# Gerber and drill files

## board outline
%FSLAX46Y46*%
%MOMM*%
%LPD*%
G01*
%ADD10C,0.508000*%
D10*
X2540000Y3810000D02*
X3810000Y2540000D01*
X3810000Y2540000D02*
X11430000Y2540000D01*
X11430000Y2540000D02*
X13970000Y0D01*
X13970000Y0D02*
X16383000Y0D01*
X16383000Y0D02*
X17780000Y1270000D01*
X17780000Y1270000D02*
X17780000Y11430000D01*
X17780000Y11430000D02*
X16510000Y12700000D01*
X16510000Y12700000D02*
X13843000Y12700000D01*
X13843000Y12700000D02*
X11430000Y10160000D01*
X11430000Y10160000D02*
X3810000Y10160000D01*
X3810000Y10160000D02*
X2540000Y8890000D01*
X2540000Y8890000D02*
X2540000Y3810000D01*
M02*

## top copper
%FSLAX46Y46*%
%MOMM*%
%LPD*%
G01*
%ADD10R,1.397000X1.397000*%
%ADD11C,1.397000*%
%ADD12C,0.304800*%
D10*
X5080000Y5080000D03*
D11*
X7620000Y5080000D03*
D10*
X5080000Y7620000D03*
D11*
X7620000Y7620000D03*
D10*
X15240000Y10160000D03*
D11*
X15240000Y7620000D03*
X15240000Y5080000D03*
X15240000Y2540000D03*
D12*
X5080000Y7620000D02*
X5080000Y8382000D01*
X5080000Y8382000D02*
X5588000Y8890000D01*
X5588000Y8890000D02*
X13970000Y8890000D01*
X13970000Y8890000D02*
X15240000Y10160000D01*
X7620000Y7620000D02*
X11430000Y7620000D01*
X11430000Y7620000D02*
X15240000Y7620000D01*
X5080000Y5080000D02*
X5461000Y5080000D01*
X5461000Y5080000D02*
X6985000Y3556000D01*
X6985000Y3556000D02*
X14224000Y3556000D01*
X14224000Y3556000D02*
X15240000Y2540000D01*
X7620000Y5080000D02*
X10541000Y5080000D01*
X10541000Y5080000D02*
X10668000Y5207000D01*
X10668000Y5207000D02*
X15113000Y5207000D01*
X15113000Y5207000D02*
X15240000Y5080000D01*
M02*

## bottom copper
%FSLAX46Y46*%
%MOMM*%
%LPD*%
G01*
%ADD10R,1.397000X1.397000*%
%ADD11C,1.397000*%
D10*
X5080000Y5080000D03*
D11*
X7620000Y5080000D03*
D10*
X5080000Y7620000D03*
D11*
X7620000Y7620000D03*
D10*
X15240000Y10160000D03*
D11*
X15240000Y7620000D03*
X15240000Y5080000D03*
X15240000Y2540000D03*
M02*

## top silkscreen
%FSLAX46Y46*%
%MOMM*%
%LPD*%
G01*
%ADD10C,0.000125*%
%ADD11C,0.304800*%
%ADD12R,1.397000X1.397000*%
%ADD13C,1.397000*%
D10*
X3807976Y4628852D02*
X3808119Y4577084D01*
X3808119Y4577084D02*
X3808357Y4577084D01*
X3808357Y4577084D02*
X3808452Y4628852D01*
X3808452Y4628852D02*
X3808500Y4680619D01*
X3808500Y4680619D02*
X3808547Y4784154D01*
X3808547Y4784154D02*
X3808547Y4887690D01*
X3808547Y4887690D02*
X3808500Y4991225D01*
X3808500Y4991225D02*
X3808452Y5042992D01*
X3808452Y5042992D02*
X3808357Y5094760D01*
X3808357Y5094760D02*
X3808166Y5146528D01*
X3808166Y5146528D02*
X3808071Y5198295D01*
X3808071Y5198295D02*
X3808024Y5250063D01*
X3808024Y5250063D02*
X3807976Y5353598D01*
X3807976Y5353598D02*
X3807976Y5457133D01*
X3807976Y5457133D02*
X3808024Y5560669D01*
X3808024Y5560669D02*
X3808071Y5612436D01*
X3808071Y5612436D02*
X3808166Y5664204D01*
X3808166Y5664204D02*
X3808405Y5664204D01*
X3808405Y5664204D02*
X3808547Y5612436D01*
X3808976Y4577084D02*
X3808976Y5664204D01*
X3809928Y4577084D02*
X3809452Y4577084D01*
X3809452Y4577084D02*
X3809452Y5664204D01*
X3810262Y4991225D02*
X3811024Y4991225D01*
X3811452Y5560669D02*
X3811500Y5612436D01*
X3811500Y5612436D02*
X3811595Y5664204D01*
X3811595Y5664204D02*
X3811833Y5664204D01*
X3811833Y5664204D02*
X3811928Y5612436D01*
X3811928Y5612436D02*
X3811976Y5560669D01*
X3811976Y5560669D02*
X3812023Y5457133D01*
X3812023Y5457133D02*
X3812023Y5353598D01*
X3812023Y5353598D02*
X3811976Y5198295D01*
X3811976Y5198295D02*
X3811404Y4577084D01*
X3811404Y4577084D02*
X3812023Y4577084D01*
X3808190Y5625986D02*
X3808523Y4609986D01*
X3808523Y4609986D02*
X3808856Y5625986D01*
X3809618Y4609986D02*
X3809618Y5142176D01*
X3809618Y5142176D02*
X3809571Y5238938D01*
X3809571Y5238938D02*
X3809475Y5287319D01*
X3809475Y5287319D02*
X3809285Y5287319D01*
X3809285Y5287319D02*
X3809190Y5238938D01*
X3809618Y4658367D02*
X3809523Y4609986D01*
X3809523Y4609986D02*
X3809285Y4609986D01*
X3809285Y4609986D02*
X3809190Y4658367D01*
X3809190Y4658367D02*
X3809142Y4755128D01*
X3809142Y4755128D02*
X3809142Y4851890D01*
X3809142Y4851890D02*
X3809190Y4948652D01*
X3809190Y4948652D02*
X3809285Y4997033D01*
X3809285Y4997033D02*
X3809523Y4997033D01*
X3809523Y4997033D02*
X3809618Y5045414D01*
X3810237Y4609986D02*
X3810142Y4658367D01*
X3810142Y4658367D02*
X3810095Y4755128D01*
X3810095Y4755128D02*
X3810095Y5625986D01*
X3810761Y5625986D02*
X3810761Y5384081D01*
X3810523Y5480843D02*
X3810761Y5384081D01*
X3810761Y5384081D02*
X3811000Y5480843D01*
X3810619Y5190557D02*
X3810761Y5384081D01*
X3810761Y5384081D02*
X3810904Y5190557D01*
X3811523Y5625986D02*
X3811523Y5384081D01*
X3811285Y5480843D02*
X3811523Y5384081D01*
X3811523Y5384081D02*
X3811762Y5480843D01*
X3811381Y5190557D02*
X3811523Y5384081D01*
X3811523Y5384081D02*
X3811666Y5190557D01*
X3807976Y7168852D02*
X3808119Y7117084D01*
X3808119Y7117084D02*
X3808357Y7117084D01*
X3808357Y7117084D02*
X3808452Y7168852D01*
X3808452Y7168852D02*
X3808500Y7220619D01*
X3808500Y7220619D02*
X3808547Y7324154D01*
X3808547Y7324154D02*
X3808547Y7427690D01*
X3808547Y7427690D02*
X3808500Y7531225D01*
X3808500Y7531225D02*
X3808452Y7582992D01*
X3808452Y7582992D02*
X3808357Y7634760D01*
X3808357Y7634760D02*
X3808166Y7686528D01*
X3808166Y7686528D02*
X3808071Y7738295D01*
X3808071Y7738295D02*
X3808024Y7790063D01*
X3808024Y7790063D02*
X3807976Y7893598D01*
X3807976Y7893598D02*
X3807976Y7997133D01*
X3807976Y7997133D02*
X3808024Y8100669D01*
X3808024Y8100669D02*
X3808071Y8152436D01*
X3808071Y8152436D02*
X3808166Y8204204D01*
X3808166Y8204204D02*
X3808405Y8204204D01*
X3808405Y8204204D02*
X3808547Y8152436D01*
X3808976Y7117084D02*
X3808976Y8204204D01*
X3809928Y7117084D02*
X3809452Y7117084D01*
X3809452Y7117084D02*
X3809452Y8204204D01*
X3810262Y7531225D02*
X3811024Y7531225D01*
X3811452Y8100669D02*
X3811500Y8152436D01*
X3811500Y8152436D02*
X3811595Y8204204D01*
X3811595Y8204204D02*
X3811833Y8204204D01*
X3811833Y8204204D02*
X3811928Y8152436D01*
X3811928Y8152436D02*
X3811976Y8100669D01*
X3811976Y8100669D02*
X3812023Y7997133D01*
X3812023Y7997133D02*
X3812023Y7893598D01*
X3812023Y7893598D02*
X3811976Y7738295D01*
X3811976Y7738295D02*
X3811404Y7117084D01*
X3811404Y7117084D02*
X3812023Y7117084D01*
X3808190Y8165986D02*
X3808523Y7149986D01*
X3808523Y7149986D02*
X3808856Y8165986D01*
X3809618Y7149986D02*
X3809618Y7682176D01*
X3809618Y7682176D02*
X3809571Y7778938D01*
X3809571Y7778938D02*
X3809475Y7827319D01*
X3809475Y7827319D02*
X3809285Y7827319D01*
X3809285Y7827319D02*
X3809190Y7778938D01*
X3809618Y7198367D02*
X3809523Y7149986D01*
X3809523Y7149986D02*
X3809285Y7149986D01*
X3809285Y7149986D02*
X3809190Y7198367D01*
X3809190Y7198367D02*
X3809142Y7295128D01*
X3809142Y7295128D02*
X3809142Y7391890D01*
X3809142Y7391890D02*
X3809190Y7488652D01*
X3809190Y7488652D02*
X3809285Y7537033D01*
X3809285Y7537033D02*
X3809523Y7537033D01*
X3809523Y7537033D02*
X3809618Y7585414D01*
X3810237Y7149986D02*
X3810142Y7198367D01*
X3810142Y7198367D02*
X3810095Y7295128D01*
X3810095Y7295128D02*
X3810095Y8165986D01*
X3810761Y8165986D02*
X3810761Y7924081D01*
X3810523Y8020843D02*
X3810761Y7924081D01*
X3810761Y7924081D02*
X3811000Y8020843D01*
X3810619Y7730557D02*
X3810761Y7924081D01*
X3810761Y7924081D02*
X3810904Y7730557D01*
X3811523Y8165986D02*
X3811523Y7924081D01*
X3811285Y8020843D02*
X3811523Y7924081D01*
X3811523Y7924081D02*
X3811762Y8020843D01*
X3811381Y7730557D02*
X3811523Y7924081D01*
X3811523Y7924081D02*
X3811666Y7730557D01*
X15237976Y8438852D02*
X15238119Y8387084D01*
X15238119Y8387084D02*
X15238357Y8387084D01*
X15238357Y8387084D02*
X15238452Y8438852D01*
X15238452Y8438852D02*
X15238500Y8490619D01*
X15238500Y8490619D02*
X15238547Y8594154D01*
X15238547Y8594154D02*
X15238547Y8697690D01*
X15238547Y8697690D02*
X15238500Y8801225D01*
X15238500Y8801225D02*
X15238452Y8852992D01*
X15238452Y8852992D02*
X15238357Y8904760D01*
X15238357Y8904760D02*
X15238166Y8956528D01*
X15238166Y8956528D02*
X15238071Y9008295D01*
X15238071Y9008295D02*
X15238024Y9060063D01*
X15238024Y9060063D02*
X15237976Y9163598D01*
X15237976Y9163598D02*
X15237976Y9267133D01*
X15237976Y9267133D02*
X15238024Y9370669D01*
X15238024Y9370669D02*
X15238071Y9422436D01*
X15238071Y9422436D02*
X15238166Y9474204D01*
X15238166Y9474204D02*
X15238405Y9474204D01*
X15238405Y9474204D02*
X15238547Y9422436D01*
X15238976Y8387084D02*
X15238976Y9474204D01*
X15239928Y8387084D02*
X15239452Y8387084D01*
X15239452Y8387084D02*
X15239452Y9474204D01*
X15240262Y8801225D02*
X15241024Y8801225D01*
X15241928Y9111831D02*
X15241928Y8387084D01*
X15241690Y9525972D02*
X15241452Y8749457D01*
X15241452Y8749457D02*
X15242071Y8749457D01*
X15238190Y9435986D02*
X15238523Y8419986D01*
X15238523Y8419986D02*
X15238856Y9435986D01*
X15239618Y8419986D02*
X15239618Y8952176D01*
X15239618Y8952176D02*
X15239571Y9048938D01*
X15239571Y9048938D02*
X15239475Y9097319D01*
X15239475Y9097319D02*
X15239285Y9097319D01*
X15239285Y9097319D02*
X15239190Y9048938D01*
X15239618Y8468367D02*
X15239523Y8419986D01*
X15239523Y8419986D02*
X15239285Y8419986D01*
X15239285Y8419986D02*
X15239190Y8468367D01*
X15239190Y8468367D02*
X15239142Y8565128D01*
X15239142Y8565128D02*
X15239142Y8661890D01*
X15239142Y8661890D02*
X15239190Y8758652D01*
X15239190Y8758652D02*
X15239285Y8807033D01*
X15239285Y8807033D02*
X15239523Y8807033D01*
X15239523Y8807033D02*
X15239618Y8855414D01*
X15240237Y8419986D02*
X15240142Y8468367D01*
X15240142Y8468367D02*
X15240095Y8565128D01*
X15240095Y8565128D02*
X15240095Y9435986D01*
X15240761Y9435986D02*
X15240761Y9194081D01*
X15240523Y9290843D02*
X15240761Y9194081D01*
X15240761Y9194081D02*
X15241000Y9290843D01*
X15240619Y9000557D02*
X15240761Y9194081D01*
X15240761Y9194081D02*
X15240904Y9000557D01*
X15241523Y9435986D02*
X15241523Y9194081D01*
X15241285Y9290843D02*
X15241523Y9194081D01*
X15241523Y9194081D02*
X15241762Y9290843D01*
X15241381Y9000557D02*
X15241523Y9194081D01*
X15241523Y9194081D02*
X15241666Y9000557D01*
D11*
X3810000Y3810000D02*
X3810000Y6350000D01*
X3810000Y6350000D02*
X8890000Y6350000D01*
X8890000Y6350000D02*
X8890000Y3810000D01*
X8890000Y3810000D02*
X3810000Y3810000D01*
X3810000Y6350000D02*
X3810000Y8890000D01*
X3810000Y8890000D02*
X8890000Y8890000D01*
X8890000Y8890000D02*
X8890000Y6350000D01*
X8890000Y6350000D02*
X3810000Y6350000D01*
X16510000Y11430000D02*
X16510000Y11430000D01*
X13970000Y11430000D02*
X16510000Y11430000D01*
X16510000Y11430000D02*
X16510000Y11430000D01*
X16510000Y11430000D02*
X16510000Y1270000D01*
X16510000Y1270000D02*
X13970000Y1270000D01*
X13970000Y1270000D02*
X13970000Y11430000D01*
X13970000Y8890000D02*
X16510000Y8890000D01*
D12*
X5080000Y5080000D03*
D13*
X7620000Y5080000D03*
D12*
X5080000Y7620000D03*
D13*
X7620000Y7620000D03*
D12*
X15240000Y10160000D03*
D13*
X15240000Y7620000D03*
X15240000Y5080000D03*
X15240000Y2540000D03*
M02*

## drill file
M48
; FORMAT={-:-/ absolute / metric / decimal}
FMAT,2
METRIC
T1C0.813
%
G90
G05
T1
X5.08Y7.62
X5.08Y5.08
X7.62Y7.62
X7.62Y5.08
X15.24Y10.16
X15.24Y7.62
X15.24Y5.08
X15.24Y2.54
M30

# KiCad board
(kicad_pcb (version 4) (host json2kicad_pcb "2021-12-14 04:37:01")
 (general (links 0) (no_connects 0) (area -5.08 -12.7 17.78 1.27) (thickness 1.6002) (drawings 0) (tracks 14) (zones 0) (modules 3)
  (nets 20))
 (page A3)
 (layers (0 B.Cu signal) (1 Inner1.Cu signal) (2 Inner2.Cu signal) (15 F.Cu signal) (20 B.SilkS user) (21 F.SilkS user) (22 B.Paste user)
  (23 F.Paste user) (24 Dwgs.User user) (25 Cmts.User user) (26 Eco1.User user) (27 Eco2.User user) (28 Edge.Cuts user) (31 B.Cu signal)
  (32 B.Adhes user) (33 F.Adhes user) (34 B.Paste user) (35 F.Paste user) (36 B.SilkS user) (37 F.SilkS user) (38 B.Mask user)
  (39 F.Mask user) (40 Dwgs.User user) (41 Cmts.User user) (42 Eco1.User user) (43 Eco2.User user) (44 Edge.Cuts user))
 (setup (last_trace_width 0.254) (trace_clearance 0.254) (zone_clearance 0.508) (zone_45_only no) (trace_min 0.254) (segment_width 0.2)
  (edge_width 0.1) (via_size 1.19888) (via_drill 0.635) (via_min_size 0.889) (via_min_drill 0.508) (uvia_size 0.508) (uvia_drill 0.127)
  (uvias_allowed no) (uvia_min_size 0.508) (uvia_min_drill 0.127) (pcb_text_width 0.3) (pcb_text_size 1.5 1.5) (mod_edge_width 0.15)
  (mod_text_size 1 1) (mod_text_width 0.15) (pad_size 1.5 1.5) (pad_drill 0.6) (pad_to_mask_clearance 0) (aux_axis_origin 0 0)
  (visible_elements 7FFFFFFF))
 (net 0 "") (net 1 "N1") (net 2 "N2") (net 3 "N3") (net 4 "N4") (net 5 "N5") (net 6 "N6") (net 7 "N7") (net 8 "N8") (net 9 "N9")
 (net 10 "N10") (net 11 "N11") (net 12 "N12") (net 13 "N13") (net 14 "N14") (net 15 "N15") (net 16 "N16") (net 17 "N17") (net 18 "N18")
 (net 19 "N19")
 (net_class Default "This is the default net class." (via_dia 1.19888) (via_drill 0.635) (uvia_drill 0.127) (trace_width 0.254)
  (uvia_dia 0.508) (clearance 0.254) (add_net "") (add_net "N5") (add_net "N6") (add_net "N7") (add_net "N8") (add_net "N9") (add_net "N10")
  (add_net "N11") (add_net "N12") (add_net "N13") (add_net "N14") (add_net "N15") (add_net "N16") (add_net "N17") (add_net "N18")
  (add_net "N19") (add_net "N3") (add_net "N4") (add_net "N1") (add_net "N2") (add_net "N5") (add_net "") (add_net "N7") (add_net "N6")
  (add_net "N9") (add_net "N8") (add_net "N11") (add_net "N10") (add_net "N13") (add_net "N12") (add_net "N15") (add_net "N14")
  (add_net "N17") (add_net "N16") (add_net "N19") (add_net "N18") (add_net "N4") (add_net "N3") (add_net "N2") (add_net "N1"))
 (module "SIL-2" (layer "F.Cu") (at 6.35 -5.08 0.00)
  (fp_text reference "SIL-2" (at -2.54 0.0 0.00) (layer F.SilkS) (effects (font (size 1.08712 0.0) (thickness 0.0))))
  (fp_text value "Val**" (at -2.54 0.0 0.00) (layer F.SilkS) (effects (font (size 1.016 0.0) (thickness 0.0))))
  (fp_line (start -2.54 1.27) (end -2.54 -1.27) (layer F.SilkS) (width 0.3048))
  (fp_line (start -2.54 -1.27) (end 2.54 -1.27) (layer F.SilkS) (width 0.3048))
  (fp_line (start 2.54 -1.27) (end 2.54 1.27) (layer F.SilkS) (width 0.3048))
  (fp_line (start 2.54 1.27) (end -2.54 1.27) (layer F.SilkS) (width 0.3048))
  (pad 1 thru_hole rect (at -1.27 0.0 0.00) (size 1.397 1.397) (drill 0.8128)
   (layers "B.Cu" "Inner1.Cu" "Inner2.Cu" "F.Cu" "F.SilkS" "B.Paste" "F.Paste") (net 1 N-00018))
  (pad 2 thru_hole circle (at 1.27 0.0 0.00) (size 1.397 1.397) (drill 0.8128)
   (layers "B.Cu" "Inner1.Cu" "Inner2.Cu" "F.Cu" "F.SilkS" "B.Paste" "F.Paste") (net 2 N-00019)))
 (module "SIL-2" (layer "F.Cu") (at 6.35 -7.62 0.00)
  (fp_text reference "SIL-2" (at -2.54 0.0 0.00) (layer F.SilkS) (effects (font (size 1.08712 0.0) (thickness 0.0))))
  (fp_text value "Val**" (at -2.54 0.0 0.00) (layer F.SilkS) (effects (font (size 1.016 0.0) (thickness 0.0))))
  (fp_line (start -2.54 1.27) (end -2.54 -1.27) (layer F.SilkS) (width 0.3048))
  (fp_line (start -2.54 -1.27) (end 2.54 -1.27) (layer F.SilkS) (width 0.3048))
  (fp_line (start 2.54 -1.27) (end 2.54 1.27) (layer F.SilkS) (width 0.3048))
  (fp_line (start 2.54 1.27) (end -2.54 1.27) (layer F.SilkS) (width 0.3048))
  (pad 1 thru_hole rect (at -1.27 0.0 0.00) (size 1.397 1.397) (drill 0.8128)
   (layers "B.Cu" "Inner1.Cu" "Inner2.Cu" "F.Cu" "F.SilkS" "B.Paste" "F.Paste") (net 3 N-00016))
  (pad 2 thru_hole circle (at 1.27 0.0 0.00) (size 1.397 1.397) (drill 0.8128)
   (layers "B.Cu" "Inner1.Cu" "Inner2.Cu" "F.Cu" "F.SilkS" "B.Paste" "F.Paste") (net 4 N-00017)))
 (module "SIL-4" (layer "F.Cu") (at 15.24 -6.35 -90.00)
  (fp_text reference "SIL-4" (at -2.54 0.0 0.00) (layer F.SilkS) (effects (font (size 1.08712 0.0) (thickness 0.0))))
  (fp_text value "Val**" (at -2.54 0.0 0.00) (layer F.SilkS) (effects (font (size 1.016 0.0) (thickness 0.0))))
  (fp_line (start -5.08 -1.27) (end -5.08 -1.27) (layer F.SilkS) (width 0.3048))
  (fp_line (start -5.08 1.27) (end -5.08 -1.27) (layer F.SilkS) (width 0.3048))
  (fp_line (start -5.08 -1.27) (end -5.08 -1.27) (layer F.SilkS) (width 0.3048))
  (fp_line (start -5.08 -1.27) (end 5.08 -1.27) (layer F.SilkS) (width 0.3048))
  (fp_line (start 5.08 -1.27) (end 5.08 1.27) (layer F.SilkS) (width 0.3048))
  (fp_line (start 5.08 1.27) (end -5.08 1.27) (layer F.SilkS) (width 0.3048))
  (fp_line (start -2.54 1.27) (end -2.54 -1.27) (layer F.SilkS) (width 0.3048))
  (pad 1 thru_hole rect (at -3.81 0.0 -90.00) (size 1.397 1.397) (drill 0.8128)
   (layers "B.Cu" "Inner1.Cu" "Inner2.Cu" "F.Cu" "F.SilkS" "B.Paste" "F.Paste") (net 3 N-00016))
  (pad 2 thru_hole circle (at -1.27 0.0 -90.00) (size 1.397 1.397) (drill 0.8128)
   (layers "B.Cu" "Inner1.Cu" "Inner2.Cu" "F.Cu" "F.SilkS" "B.Paste" "F.Paste") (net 4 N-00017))
  (pad 3 thru_hole circle (at 1.27 0.0 -90.00) (size 1.397 1.397) (drill 0.8128)
   (layers "B.Cu" "Inner1.Cu" "Inner2.Cu" "F.Cu" "F.SilkS" "B.Paste" "F.Paste") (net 2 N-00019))
  (pad 4 thru_hole circle (at 3.81 0.0 -90.00) (size 1.397 1.397) (drill 0.8128)
   (layers "B.Cu" "Inner1.Cu" "Inner2.Cu" "F.Cu" "F.SilkS" "B.Paste" "F.Paste") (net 1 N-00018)))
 (segment (start 5.08 -7.62) (end 5.08 -8.382) (width 0.3048) (layer F.Cu) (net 3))
 (segment (start 5.08 -8.382) (end 5.588 -8.89) (width 0.3048) (layer F.Cu) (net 3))
 (segment (start 5.588 -8.89) (end 13.97 -8.89) (width 0.3048) (layer F.Cu) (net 3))
 (segment (start 13.97 -8.89) (end 15.24 -10.16) (width 0.3048) (layer F.Cu) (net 3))
 (segment (start 7.62 -7.62) (end 11.43 -7.62) (width 0.3048) (layer F.Cu) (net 4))
 (segment (start 11.43 -7.62) (end 15.24 -7.62) (width 0.3048) (layer F.Cu) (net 4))
 (segment (start 5.08 -5.08) (end 5.461 -5.08) (width 0.3048) (layer F.Cu) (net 1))
 (segment (start 5.461 -5.08) (end 6.985 -3.556) (width 0.3048) (layer F.Cu) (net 1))
 (segment (start 6.985 -3.556) (end 14.224 -3.556) (width 0.3048) (layer F.Cu) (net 1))
 (segment (start 14.224 -3.556) (end 15.24 -2.54) (width 0.3048) (layer F.Cu) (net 1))
 (segment (start 7.62 -5.08) (end 10.541 -5.08) (width 0.3048) (layer F.Cu) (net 2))
 (segment (start 10.541 -5.08) (end 10.668 -5.207) (width 0.3048) (layer F.Cu) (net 2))
 (segment (start 10.668 -5.207) (end 15.113 -5.207) (width 0.3048) (layer F.Cu) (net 2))
 (segment (start 15.113 -5.207) (end 15.24 -5.08) (width 0.3048) (layer F.Cu) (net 2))
 (gr_line (start 2.54 -3.81) (end 3.81 -2.54) (angle 51566.20) (width 0.508) (layer Edge.Cuts))
 (gr_line (start 3.81 -2.54) (end 11.43 -2.54) (angle 51566.20) (width 0.508) (layer Edge.Cuts))
 (gr_line (start 11.43 -2.54) (end 13.97 0.0) (angle 51566.20) (width 0.508) (layer Edge.Cuts))
 (gr_line (start 13.97 0.0) (end 16.383 0.0) (angle 51566.20) (width 0.508) (layer Edge.Cuts))
 (gr_line (start 16.383 0.0) (end 17.78 -1.27) (angle 51566.20) (width 0.508) (layer Edge.Cuts))
 (gr_line (start 17.78 -1.27) (end 17.78 -11.43) (angle 51566.20) (width 0.508) (layer Edge.Cuts))
 (gr_line (start 17.78 -11.43) (end 16.51 -12.7) (angle 51566.20) (width 0.508) (layer Edge.Cuts))
 (gr_line (start 16.51 -12.7) (end 13.843 -12.7) (angle 51566.20) (width 0.508) (layer Edge.Cuts))
 (gr_line (start 13.843 -12.7) (end 11.43 -10.16) (angle 51566.20) (width 0.508) (layer Edge.Cuts))
 (gr_line (start 11.43 -10.16) (end 3.81 -10.16) (angle 51566.20) (width 0.508) (layer Edge.Cuts))
 (gr_line (start 3.81 -10.16) (end 2.54 -8.89) (angle 51566.20) (width 0.508) (layer Edge.Cuts))
 (gr_line (start 2.54 -8.89) (end 2.54 -3.81) (angle 51566.20) (width 0.508) (layer Edge.Cuts)))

